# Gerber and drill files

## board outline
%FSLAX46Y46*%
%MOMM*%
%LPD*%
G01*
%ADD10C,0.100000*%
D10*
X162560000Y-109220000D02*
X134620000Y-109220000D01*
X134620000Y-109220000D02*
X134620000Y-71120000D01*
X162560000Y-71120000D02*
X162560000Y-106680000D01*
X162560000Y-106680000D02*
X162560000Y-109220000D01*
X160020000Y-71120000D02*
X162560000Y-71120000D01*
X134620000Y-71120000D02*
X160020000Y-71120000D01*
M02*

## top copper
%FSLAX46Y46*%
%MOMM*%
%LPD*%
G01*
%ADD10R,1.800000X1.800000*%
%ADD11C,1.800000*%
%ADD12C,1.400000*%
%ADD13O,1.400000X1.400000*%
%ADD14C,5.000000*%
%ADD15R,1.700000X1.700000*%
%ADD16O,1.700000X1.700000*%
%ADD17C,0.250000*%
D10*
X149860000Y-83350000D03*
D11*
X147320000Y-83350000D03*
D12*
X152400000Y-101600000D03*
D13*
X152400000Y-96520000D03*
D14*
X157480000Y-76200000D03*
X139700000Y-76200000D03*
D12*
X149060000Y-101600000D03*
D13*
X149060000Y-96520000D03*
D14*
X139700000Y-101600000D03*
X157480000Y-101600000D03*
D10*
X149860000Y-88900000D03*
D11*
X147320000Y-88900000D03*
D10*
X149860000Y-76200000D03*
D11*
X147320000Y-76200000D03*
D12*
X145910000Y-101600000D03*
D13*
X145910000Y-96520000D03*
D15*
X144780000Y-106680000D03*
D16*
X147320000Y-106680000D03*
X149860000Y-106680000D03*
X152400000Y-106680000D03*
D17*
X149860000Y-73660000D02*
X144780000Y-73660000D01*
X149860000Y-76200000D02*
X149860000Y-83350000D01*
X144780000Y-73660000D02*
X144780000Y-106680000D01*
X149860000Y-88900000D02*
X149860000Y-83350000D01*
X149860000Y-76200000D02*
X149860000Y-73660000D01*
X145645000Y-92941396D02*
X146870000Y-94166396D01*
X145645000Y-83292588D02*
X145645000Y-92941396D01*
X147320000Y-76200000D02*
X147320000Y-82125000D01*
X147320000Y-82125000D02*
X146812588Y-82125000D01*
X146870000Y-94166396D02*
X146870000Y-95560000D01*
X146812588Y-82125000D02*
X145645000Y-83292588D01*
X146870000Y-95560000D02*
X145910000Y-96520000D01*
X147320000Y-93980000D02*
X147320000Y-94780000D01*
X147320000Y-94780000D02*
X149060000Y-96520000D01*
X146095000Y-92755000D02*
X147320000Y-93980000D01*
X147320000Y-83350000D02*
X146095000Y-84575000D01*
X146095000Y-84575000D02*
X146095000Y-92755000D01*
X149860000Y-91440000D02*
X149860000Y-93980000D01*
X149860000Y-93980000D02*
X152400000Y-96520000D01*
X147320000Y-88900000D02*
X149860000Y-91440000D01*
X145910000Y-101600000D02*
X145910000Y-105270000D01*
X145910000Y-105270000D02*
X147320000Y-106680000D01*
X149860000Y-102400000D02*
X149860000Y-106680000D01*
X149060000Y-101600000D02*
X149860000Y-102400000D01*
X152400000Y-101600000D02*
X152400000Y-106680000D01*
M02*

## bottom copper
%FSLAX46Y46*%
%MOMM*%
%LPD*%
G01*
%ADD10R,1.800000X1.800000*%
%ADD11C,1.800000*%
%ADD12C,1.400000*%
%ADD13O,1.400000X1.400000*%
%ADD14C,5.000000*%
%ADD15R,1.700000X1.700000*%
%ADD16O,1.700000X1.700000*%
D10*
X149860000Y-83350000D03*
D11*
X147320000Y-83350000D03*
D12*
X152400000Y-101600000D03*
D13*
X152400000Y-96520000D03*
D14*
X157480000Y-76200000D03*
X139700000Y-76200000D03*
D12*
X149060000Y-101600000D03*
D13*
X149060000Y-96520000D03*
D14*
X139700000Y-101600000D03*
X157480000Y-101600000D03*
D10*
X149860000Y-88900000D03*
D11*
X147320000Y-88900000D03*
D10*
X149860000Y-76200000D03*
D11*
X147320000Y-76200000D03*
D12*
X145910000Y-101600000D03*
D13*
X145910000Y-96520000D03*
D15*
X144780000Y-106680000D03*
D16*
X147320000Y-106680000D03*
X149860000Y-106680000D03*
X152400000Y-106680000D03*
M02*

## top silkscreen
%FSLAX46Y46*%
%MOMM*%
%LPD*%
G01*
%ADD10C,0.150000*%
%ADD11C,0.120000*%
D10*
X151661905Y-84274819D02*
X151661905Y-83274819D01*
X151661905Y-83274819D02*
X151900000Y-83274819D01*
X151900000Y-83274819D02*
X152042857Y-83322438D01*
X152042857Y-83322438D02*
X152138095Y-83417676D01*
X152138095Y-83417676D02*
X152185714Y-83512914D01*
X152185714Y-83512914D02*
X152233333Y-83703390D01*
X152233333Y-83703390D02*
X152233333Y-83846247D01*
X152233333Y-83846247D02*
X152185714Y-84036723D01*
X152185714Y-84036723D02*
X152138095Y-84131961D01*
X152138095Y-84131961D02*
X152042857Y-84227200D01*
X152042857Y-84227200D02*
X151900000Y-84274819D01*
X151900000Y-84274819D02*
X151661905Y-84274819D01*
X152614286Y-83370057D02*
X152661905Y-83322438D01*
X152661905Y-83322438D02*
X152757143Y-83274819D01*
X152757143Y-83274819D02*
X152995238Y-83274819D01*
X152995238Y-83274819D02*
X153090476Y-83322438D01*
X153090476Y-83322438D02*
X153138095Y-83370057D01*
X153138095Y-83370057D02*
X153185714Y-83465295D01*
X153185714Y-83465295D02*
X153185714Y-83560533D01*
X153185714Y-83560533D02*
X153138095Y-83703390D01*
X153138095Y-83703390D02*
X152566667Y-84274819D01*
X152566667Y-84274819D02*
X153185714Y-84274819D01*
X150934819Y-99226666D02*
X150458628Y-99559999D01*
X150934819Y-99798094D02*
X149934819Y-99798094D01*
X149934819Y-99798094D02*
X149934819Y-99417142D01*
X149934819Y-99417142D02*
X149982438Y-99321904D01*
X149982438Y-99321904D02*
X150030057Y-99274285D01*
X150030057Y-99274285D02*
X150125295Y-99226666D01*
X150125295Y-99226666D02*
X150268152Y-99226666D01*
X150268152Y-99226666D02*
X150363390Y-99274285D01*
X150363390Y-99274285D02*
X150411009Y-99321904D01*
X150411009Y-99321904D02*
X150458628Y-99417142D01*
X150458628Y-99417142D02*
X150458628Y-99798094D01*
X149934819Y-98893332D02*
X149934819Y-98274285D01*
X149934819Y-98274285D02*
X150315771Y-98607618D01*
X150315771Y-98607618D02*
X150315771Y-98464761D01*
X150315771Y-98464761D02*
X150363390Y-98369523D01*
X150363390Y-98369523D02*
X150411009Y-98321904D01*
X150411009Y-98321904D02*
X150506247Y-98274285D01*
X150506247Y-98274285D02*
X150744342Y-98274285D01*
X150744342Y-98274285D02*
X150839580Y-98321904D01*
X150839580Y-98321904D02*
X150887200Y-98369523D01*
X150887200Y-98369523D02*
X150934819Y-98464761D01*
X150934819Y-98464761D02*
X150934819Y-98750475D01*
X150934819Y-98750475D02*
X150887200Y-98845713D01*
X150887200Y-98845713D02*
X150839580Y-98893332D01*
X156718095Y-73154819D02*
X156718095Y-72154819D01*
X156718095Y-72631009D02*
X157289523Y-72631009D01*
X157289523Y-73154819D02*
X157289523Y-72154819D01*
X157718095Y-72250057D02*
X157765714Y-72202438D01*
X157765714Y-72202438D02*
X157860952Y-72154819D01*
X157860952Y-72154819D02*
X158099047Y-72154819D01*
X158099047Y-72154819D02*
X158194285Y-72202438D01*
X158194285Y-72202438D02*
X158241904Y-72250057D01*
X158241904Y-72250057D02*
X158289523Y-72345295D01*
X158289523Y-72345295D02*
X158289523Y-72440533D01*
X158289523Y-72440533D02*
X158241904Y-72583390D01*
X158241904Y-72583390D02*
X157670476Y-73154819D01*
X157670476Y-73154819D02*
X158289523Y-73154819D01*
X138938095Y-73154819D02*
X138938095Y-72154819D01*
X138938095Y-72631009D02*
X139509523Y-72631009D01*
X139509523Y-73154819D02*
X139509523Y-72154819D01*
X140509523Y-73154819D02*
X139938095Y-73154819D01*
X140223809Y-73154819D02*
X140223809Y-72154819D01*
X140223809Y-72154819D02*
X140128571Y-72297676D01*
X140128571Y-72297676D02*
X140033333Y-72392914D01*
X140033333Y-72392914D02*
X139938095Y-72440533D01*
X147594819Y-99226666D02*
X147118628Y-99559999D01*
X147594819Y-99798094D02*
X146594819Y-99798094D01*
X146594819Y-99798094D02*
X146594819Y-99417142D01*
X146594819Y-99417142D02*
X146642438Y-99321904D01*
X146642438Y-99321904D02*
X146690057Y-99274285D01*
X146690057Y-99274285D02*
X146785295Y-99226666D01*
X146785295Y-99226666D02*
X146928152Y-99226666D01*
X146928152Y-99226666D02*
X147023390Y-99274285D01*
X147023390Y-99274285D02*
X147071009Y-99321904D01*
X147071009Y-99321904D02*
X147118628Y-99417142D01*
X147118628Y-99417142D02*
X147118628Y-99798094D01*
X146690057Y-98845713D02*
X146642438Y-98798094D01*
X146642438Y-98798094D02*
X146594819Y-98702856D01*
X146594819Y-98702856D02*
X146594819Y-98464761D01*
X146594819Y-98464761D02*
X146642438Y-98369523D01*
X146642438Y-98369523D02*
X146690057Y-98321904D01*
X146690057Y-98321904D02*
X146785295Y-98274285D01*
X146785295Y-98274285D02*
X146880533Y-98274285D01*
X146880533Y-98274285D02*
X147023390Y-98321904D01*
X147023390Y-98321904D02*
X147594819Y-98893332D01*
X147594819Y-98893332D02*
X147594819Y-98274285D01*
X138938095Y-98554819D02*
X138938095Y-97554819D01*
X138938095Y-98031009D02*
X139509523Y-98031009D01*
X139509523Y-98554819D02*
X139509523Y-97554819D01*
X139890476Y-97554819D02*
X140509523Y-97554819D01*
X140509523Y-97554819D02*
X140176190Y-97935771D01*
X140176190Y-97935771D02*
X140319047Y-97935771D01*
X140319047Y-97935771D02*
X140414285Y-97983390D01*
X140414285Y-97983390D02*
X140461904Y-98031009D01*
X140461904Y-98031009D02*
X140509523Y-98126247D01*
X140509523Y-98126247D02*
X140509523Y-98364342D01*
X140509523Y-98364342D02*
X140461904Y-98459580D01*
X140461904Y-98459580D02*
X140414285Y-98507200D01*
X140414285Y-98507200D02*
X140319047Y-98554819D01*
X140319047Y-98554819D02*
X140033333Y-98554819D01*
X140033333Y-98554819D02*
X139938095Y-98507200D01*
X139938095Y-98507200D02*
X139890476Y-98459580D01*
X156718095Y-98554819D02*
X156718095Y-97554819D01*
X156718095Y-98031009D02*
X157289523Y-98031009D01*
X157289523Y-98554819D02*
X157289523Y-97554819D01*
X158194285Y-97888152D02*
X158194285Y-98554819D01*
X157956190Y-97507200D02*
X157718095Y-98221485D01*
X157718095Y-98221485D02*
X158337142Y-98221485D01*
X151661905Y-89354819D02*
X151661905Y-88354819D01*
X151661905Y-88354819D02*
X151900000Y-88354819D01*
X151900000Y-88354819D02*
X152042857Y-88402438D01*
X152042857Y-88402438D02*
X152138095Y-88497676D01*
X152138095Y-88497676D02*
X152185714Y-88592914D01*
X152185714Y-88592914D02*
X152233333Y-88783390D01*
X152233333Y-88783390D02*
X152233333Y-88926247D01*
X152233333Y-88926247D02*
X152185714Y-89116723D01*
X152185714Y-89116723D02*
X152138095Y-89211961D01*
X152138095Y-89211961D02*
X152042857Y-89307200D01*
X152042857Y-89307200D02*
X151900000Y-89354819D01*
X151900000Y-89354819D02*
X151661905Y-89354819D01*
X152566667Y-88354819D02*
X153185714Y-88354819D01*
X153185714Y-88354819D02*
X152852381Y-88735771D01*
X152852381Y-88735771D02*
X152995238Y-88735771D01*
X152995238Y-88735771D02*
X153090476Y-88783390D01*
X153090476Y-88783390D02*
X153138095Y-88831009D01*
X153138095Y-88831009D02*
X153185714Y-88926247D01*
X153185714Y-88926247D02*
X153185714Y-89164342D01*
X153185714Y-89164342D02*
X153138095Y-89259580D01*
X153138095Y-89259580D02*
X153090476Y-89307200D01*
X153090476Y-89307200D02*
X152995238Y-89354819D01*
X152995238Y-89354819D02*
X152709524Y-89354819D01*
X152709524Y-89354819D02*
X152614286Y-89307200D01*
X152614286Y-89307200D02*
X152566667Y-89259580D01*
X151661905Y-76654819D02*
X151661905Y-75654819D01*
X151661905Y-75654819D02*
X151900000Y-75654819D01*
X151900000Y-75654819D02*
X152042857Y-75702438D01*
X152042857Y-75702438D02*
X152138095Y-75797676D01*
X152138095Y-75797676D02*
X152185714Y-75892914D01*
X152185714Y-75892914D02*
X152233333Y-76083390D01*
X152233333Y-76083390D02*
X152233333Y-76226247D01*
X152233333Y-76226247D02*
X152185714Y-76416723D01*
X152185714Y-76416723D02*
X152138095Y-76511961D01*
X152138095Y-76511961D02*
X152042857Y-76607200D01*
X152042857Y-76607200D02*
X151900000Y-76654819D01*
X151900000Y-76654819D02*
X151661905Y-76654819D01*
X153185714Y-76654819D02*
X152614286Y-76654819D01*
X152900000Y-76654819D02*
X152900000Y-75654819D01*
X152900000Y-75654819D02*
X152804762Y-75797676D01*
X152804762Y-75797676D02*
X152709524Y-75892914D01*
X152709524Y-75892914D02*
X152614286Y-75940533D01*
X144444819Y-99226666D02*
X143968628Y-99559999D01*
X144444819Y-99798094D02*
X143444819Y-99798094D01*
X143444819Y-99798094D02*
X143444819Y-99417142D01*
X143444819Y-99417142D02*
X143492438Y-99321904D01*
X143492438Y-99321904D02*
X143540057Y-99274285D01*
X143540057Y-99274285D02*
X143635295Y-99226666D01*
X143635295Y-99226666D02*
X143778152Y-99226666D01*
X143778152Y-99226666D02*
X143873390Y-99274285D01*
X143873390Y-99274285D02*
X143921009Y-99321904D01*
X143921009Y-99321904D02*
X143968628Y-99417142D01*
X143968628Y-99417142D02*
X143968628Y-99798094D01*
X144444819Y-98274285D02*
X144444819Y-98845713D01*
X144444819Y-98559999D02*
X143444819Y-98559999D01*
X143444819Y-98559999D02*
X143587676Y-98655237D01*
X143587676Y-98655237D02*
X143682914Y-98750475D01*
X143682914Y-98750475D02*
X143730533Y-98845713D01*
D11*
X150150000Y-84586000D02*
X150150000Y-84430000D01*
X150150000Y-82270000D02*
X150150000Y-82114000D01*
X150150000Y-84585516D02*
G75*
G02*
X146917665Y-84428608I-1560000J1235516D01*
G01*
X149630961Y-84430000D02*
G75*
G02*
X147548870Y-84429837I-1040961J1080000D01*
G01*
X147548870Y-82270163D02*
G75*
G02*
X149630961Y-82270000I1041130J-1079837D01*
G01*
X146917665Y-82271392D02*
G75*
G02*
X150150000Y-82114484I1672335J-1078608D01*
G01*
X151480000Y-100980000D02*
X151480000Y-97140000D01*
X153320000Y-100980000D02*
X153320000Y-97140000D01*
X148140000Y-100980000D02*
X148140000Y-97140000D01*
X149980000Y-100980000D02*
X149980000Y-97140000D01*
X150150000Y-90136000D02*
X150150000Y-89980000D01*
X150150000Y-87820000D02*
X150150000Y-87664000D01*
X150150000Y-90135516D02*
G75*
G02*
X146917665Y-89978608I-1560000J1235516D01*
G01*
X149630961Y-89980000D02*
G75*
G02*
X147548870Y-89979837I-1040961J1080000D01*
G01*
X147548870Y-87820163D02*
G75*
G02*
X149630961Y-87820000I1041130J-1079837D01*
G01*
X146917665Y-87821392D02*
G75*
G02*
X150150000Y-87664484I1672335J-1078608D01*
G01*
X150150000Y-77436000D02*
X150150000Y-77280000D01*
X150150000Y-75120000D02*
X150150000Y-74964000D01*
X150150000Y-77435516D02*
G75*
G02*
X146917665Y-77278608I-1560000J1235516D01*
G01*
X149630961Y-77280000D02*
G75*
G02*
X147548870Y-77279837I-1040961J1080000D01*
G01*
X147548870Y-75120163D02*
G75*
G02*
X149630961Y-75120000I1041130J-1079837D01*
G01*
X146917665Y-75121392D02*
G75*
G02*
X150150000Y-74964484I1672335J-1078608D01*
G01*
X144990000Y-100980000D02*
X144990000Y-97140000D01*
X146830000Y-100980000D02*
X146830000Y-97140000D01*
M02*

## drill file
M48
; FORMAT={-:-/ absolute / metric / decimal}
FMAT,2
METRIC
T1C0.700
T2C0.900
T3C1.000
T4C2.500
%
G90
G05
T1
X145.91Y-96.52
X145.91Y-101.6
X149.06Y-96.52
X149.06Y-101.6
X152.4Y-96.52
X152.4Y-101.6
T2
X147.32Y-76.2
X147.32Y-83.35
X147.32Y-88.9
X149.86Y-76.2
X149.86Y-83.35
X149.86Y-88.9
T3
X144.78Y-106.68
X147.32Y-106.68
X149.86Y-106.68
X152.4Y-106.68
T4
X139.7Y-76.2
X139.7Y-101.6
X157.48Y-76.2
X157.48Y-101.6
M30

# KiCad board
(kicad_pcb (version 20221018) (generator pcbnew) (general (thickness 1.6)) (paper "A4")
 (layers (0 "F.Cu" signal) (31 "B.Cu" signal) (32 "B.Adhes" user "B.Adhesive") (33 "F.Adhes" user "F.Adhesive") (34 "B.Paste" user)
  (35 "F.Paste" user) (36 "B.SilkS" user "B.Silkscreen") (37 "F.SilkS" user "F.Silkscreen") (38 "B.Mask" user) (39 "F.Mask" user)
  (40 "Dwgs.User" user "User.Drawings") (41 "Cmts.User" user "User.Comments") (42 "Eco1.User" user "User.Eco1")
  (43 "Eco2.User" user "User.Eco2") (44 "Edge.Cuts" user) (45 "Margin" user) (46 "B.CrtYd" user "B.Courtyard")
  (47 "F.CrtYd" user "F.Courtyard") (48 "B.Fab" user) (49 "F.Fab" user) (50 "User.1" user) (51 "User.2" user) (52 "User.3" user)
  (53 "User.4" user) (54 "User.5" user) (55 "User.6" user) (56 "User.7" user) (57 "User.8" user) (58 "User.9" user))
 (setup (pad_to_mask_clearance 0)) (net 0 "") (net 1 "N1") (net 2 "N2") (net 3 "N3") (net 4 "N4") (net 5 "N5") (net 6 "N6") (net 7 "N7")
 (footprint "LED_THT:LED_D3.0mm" (layer "F.Cu") (at 149.86 83.35 180)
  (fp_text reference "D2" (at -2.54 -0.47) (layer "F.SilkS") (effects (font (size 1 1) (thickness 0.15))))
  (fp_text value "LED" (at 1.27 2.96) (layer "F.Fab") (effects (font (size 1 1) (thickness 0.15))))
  (fp_line (start -0.29 -1.236) (end -0.29 -1.08) (stroke (width 0.12) (type solid)) (layer "F.SilkS"))
  (fp_line (start -0.29 1.08) (end -0.29 1.236) (stroke (width 0.12) (type solid)) (layer "F.SilkS"))
  (fp_arc (start -0.29 -1.235516) (mid 1.366487 -1.987659) (end 2.942335 -1.078608) (stroke (width 0.12) (type solid)) (layer "F.SilkS"))
  (fp_arc (start 0.229039 -1.08) (mid 1.270117 -1.5) (end 2.31113 -1.079837) (stroke (width 0.12) (type solid)) (layer "F.SilkS"))
  (fp_arc (start 2.31113 1.079837) (mid 1.270117 1.5) (end 0.229039 1.08) (stroke (width 0.12) (type solid)) (layer "F.SilkS"))
  (fp_arc (start 2.942335 1.078608) (mid 1.366487 1.987659) (end -0.29 1.235516) (stroke (width 0.12) (type solid)) (layer "F.SilkS"))
  (pad "1" thru_hole rect (at 0 0 180) (size 1.8 1.8) (drill 0.9) (layers "*.Cu" "*.Mask") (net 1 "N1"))
  (pad "2" thru_hole circle (at 2.54 0 180) (size 1.8 1.8) (drill 0.9) (layers "*.Cu" "*.Mask") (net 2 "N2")))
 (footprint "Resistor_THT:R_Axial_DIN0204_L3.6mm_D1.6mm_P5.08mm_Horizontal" (layer "F.Cu") (at 152.4 101.6 90)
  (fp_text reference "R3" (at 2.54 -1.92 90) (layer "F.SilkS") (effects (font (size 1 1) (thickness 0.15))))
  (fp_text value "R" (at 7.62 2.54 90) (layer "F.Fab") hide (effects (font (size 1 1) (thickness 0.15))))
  (fp_line (start 0.62 -0.92) (end 4.46 -0.92) (stroke (width 0.12) (type solid)) (layer "F.SilkS"))
  (fp_line (start 0.62 0.92) (end 4.46 0.92) (stroke (width 0.12) (type solid)) (layer "F.SilkS"))
  (pad "1" thru_hole circle (at 0 0 90) (size 1.4 1.4) (drill 0.7) (layers "*.Cu" "*.Mask") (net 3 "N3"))
  (pad "2" thru_hole oval (at 5.08 0 90) (size 1.4 1.4) (drill 0.7) (layers "*.Cu" "*.Mask") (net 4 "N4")))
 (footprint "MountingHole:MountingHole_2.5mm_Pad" (layer "F.Cu") (at 157.48 76.2)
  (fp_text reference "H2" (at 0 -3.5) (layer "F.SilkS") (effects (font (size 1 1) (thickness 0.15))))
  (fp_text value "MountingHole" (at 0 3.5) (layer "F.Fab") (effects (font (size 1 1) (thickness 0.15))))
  (pad "1" thru_hole circle (at 0 0) (size 5 5) (drill 2.5) (layers "*.Cu" "*.Mask")))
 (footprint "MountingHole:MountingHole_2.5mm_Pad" (layer "F.Cu") (at 139.7 76.2)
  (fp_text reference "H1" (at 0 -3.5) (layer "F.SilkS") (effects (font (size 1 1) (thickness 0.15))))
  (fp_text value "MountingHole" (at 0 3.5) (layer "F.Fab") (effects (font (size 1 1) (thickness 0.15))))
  (pad "1" thru_hole circle (at 0 0) (size 5 5) (drill 2.5) (layers "*.Cu" "*.Mask")))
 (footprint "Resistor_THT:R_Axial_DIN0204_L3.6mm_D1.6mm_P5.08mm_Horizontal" (layer "F.Cu") (at 149.06 101.6 90)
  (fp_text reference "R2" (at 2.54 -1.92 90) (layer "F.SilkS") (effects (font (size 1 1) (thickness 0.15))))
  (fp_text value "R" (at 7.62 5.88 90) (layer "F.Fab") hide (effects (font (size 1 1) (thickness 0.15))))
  (fp_line (start 0.62 -0.92) (end 4.46 -0.92) (stroke (width 0.12) (type solid)) (layer "F.SilkS"))
  (fp_line (start 0.62 0.92) (end 4.46 0.92) (stroke (width 0.12) (type solid)) (layer "F.SilkS"))
  (pad "1" thru_hole circle (at 0 0 90) (size 1.4 1.4) (drill 0.7) (layers "*.Cu" "*.Mask") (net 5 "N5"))
  (pad "2" thru_hole oval (at 5.08 0 90) (size 1.4 1.4) (drill 0.7) (layers "*.Cu" "*.Mask") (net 2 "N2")))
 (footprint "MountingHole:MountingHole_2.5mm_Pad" (layer "F.Cu") (at 139.7 101.6)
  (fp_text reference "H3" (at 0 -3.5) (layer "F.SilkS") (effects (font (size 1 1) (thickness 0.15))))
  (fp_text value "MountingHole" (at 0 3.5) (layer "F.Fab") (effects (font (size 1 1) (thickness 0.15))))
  (pad "1" thru_hole circle (at 0 0) (size 5 5) (drill 2.5) (layers "*.Cu" "*.Mask")))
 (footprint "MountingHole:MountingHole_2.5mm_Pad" (layer "F.Cu") (at 157.48 101.6)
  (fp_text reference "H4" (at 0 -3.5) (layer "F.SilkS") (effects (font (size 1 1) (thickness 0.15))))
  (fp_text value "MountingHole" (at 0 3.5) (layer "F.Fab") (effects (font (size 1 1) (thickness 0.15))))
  (pad "1" thru_hole circle (at 0 0) (size 5 5) (drill 2.5) (layers "*.Cu" "*.Mask")))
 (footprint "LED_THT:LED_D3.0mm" (layer "F.Cu") (at 149.86 88.9 180)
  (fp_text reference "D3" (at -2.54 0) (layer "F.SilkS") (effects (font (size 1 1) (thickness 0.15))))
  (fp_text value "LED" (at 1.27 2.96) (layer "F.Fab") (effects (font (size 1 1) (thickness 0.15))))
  (fp_line (start -0.29 -1.236) (end -0.29 -1.08) (stroke (width 0.12) (type solid)) (layer "F.SilkS"))
  (fp_line (start -0.29 1.08) (end -0.29 1.236) (stroke (width 0.12) (type solid)) (layer "F.SilkS"))
  (fp_arc (start -0.29 -1.235516) (mid 1.366487 -1.987659) (end 2.942335 -1.078608) (stroke (width 0.12) (type solid)) (layer "F.SilkS"))
  (fp_arc (start 0.229039 -1.08) (mid 1.270117 -1.5) (end 2.31113 -1.079837) (stroke (width 0.12) (type solid)) (layer "F.SilkS"))
  (fp_arc (start 2.31113 1.079837) (mid 1.270117 1.5) (end 0.229039 1.08) (stroke (width 0.12) (type solid)) (layer "F.SilkS"))
  (fp_arc (start 2.942335 1.078608) (mid 1.366487 1.987659) (end -0.29 1.235516) (stroke (width 0.12) (type solid)) (layer "F.SilkS"))
  (pad "1" thru_hole rect (at 0 0 180) (size 1.8 1.8) (drill 0.9) (layers "*.Cu" "*.Mask") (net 1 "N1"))
  (pad "2" thru_hole circle (at 2.54 0 180) (size 1.8 1.8) (drill 0.9) (layers "*.Cu" "*.Mask") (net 4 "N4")))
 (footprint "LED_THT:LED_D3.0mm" (layer "F.Cu") (at 149.86 76.2 180)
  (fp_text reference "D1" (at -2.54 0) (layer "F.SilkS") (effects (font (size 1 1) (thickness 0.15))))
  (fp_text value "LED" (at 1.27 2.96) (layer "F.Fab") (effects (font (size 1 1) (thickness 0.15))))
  (fp_line (start -0.29 -1.236) (end -0.29 -1.08) (stroke (width 0.12) (type solid)) (layer "F.SilkS"))
  (fp_line (start -0.29 1.08) (end -0.29 1.236) (stroke (width 0.12) (type solid)) (layer "F.SilkS"))
  (fp_arc (start -0.29 -1.235516) (mid 1.366487 -1.987659) (end 2.942335 -1.078608) (stroke (width 0.12) (type solid)) (layer "F.SilkS"))
  (fp_arc (start 0.229039 -1.08) (mid 1.270117 -1.5) (end 2.31113 -1.079837) (stroke (width 0.12) (type solid)) (layer "F.SilkS"))
  (fp_arc (start 2.31113 1.079837) (mid 1.270117 1.5) (end 0.229039 1.08) (stroke (width 0.12) (type solid)) (layer "F.SilkS"))
  (fp_arc (start 2.942335 1.078608) (mid 1.366487 1.987659) (end -0.29 1.235516) (stroke (width 0.12) (type solid)) (layer "F.SilkS"))
  (pad "1" thru_hole rect (at 0 0 180) (size 1.8 1.8) (drill 0.9) (layers "*.Cu" "*.Mask") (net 1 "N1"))
  (pad "2" thru_hole circle (at 2.54 0 180) (size 1.8 1.8) (drill 0.9) (layers "*.Cu" "*.Mask") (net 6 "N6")))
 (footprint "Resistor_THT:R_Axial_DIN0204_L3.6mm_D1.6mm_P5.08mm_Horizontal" (layer "F.Cu") (at 145.91 101.6 90)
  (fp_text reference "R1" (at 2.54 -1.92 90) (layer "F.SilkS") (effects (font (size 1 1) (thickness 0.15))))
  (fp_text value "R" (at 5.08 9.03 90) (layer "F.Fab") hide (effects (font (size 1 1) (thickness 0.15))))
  (fp_line (start 0.62 -0.92) (end 4.46 -0.92) (stroke (width 0.12) (type solid)) (layer "F.SilkS"))
  (fp_line (start 0.62 0.92) (end 4.46 0.92) (stroke (width 0.12) (type solid)) (layer "F.SilkS"))
  (pad "1" thru_hole circle (at 0 0 90) (size 1.4 1.4) (drill 0.7) (layers "*.Cu" "*.Mask") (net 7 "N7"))
  (pad "2" thru_hole oval (at 5.08 0 90) (size 1.4 1.4) (drill 0.7) (layers "*.Cu" "*.Mask") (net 6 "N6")))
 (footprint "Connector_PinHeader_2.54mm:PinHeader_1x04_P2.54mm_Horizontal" (layer "B.Cu") (at 144.78 106.68 -90)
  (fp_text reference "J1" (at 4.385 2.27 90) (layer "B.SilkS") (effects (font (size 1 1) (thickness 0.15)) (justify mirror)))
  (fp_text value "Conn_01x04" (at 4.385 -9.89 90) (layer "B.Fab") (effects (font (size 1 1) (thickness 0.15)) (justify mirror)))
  (pad "1" thru_hole rect (at 0 0 270) (size 1.7 1.7) (drill 1) (layers "*.Cu" "*.Mask") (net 1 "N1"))
  (pad "2" thru_hole oval (at 0 -2.54 270) (size 1.7 1.7) (drill 1) (layers "*.Cu" "*.Mask") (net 7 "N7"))
  (pad "3" thru_hole oval (at 0 -5.08 270) (size 1.7 1.7) (drill 1) (layers "*.Cu" "*.Mask") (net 5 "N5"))
  (pad "4" thru_hole oval (at 0 -7.62 270) (size 1.7 1.7) (drill 1) (layers "*.Cu" "*.Mask") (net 3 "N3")))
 (gr_line (start 162.56 109.22) (end 134.62 109.22) (stroke (width 0.1) (type default)) (layer "Edge.Cuts"))
 (gr_line (start 134.62 109.22) (end 134.62 71.12) (stroke (width 0.1) (type default)) (layer "Edge.Cuts"))
 (gr_line (start 162.56 71.12) (end 162.56 106.68) (stroke (width 0.1) (type default)) (layer "Edge.Cuts"))
 (gr_line (start 162.56 106.68) (end 162.56 109.22) (stroke (width 0.1) (type default)) (layer "Edge.Cuts"))
 (gr_line (start 160.02 71.12) (end 162.56 71.12) (stroke (width 0.1) (type default)) (layer "Edge.Cuts"))
 (gr_line (start 134.62 71.12) (end 160.02 71.12) (stroke (width 0.1) (type default)) (layer "Edge.Cuts"))
 (segment (start 149.86 73.66) (end 144.78 73.66) (width 0.25) (layer "F.Cu") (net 1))
 (segment (start 149.86 76.2) (end 149.86 83.35) (width 0.25) (layer "F.Cu") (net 1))
 (segment (start 144.78 73.66) (end 144.78 106.68) (width 0.25) (layer "F.Cu") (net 1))
 (segment (start 149.86 88.9) (end 149.86 83.35) (width 0.25) (layer "F.Cu") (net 1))
 (segment (start 149.86 76.2) (end 149.86 73.66) (width 0.25) (layer "F.Cu") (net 1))
 (segment (start 145.645 92.941396) (end 146.87 94.166396) (width 0.25) (layer "F.Cu") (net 6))
 (segment (start 145.645 83.292588) (end 145.645 92.941396) (width 0.25) (layer "F.Cu") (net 6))
 (segment (start 147.32 76.2) (end 147.32 82.125) (width 0.25) (layer "F.Cu") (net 6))
 (segment (start 147.32 82.125) (end 146.812588 82.125) (width 0.25) (layer "F.Cu") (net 6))
 (segment (start 146.87 94.166396) (end 146.87 95.56) (width 0.25) (layer "F.Cu") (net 6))
 (segment (start 146.812588 82.125) (end 145.645 83.292588) (width 0.25) (layer "F.Cu") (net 6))
 (segment (start 146.87 95.56) (end 145.91 96.52) (width 0.25) (layer "F.Cu") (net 6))
 (segment (start 147.32 93.98) (end 147.32 94.78) (width 0.25) (layer "F.Cu") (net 2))
 (segment (start 147.32 94.78) (end 149.06 96.52) (width 0.25) (layer "F.Cu") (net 2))
 (segment (start 146.095 92.755) (end 147.32 93.98) (width 0.25) (layer "F.Cu") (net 2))
 (segment (start 147.32 83.35) (end 146.095 84.575) (width 0.25) (layer "F.Cu") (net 2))
 (segment (start 146.095 84.575) (end 146.095 92.755) (width 0.25) (layer "F.Cu") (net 2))
 (segment (start 149.86 91.44) (end 149.86 93.98) (width 0.25) (layer "F.Cu") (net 4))
 (segment (start 149.86 93.98) (end 152.4 96.52) (width 0.25) (layer "F.Cu") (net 4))
 (segment (start 147.32 88.9) (end 149.86 91.44) (width 0.25) (layer "F.Cu") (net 4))
 (segment (start 145.91 101.6) (end 145.91 105.27) (width 0.25) (layer "F.Cu") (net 7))
 (segment (start 145.91 105.27) (end 147.32 106.68) (width 0.25) (layer "F.Cu") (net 7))
 (segment (start 149.86 102.4) (end 149.86 106.68) (width 0.25) (layer "F.Cu") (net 5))
 (segment (start 149.06 101.6) (end 149.86 102.4) (width 0.25) (layer "F.Cu") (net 5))
 (segment (start 152.4 101.6) (end 152.4 106.68) (width 0.25) (layer "F.Cu") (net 3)))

